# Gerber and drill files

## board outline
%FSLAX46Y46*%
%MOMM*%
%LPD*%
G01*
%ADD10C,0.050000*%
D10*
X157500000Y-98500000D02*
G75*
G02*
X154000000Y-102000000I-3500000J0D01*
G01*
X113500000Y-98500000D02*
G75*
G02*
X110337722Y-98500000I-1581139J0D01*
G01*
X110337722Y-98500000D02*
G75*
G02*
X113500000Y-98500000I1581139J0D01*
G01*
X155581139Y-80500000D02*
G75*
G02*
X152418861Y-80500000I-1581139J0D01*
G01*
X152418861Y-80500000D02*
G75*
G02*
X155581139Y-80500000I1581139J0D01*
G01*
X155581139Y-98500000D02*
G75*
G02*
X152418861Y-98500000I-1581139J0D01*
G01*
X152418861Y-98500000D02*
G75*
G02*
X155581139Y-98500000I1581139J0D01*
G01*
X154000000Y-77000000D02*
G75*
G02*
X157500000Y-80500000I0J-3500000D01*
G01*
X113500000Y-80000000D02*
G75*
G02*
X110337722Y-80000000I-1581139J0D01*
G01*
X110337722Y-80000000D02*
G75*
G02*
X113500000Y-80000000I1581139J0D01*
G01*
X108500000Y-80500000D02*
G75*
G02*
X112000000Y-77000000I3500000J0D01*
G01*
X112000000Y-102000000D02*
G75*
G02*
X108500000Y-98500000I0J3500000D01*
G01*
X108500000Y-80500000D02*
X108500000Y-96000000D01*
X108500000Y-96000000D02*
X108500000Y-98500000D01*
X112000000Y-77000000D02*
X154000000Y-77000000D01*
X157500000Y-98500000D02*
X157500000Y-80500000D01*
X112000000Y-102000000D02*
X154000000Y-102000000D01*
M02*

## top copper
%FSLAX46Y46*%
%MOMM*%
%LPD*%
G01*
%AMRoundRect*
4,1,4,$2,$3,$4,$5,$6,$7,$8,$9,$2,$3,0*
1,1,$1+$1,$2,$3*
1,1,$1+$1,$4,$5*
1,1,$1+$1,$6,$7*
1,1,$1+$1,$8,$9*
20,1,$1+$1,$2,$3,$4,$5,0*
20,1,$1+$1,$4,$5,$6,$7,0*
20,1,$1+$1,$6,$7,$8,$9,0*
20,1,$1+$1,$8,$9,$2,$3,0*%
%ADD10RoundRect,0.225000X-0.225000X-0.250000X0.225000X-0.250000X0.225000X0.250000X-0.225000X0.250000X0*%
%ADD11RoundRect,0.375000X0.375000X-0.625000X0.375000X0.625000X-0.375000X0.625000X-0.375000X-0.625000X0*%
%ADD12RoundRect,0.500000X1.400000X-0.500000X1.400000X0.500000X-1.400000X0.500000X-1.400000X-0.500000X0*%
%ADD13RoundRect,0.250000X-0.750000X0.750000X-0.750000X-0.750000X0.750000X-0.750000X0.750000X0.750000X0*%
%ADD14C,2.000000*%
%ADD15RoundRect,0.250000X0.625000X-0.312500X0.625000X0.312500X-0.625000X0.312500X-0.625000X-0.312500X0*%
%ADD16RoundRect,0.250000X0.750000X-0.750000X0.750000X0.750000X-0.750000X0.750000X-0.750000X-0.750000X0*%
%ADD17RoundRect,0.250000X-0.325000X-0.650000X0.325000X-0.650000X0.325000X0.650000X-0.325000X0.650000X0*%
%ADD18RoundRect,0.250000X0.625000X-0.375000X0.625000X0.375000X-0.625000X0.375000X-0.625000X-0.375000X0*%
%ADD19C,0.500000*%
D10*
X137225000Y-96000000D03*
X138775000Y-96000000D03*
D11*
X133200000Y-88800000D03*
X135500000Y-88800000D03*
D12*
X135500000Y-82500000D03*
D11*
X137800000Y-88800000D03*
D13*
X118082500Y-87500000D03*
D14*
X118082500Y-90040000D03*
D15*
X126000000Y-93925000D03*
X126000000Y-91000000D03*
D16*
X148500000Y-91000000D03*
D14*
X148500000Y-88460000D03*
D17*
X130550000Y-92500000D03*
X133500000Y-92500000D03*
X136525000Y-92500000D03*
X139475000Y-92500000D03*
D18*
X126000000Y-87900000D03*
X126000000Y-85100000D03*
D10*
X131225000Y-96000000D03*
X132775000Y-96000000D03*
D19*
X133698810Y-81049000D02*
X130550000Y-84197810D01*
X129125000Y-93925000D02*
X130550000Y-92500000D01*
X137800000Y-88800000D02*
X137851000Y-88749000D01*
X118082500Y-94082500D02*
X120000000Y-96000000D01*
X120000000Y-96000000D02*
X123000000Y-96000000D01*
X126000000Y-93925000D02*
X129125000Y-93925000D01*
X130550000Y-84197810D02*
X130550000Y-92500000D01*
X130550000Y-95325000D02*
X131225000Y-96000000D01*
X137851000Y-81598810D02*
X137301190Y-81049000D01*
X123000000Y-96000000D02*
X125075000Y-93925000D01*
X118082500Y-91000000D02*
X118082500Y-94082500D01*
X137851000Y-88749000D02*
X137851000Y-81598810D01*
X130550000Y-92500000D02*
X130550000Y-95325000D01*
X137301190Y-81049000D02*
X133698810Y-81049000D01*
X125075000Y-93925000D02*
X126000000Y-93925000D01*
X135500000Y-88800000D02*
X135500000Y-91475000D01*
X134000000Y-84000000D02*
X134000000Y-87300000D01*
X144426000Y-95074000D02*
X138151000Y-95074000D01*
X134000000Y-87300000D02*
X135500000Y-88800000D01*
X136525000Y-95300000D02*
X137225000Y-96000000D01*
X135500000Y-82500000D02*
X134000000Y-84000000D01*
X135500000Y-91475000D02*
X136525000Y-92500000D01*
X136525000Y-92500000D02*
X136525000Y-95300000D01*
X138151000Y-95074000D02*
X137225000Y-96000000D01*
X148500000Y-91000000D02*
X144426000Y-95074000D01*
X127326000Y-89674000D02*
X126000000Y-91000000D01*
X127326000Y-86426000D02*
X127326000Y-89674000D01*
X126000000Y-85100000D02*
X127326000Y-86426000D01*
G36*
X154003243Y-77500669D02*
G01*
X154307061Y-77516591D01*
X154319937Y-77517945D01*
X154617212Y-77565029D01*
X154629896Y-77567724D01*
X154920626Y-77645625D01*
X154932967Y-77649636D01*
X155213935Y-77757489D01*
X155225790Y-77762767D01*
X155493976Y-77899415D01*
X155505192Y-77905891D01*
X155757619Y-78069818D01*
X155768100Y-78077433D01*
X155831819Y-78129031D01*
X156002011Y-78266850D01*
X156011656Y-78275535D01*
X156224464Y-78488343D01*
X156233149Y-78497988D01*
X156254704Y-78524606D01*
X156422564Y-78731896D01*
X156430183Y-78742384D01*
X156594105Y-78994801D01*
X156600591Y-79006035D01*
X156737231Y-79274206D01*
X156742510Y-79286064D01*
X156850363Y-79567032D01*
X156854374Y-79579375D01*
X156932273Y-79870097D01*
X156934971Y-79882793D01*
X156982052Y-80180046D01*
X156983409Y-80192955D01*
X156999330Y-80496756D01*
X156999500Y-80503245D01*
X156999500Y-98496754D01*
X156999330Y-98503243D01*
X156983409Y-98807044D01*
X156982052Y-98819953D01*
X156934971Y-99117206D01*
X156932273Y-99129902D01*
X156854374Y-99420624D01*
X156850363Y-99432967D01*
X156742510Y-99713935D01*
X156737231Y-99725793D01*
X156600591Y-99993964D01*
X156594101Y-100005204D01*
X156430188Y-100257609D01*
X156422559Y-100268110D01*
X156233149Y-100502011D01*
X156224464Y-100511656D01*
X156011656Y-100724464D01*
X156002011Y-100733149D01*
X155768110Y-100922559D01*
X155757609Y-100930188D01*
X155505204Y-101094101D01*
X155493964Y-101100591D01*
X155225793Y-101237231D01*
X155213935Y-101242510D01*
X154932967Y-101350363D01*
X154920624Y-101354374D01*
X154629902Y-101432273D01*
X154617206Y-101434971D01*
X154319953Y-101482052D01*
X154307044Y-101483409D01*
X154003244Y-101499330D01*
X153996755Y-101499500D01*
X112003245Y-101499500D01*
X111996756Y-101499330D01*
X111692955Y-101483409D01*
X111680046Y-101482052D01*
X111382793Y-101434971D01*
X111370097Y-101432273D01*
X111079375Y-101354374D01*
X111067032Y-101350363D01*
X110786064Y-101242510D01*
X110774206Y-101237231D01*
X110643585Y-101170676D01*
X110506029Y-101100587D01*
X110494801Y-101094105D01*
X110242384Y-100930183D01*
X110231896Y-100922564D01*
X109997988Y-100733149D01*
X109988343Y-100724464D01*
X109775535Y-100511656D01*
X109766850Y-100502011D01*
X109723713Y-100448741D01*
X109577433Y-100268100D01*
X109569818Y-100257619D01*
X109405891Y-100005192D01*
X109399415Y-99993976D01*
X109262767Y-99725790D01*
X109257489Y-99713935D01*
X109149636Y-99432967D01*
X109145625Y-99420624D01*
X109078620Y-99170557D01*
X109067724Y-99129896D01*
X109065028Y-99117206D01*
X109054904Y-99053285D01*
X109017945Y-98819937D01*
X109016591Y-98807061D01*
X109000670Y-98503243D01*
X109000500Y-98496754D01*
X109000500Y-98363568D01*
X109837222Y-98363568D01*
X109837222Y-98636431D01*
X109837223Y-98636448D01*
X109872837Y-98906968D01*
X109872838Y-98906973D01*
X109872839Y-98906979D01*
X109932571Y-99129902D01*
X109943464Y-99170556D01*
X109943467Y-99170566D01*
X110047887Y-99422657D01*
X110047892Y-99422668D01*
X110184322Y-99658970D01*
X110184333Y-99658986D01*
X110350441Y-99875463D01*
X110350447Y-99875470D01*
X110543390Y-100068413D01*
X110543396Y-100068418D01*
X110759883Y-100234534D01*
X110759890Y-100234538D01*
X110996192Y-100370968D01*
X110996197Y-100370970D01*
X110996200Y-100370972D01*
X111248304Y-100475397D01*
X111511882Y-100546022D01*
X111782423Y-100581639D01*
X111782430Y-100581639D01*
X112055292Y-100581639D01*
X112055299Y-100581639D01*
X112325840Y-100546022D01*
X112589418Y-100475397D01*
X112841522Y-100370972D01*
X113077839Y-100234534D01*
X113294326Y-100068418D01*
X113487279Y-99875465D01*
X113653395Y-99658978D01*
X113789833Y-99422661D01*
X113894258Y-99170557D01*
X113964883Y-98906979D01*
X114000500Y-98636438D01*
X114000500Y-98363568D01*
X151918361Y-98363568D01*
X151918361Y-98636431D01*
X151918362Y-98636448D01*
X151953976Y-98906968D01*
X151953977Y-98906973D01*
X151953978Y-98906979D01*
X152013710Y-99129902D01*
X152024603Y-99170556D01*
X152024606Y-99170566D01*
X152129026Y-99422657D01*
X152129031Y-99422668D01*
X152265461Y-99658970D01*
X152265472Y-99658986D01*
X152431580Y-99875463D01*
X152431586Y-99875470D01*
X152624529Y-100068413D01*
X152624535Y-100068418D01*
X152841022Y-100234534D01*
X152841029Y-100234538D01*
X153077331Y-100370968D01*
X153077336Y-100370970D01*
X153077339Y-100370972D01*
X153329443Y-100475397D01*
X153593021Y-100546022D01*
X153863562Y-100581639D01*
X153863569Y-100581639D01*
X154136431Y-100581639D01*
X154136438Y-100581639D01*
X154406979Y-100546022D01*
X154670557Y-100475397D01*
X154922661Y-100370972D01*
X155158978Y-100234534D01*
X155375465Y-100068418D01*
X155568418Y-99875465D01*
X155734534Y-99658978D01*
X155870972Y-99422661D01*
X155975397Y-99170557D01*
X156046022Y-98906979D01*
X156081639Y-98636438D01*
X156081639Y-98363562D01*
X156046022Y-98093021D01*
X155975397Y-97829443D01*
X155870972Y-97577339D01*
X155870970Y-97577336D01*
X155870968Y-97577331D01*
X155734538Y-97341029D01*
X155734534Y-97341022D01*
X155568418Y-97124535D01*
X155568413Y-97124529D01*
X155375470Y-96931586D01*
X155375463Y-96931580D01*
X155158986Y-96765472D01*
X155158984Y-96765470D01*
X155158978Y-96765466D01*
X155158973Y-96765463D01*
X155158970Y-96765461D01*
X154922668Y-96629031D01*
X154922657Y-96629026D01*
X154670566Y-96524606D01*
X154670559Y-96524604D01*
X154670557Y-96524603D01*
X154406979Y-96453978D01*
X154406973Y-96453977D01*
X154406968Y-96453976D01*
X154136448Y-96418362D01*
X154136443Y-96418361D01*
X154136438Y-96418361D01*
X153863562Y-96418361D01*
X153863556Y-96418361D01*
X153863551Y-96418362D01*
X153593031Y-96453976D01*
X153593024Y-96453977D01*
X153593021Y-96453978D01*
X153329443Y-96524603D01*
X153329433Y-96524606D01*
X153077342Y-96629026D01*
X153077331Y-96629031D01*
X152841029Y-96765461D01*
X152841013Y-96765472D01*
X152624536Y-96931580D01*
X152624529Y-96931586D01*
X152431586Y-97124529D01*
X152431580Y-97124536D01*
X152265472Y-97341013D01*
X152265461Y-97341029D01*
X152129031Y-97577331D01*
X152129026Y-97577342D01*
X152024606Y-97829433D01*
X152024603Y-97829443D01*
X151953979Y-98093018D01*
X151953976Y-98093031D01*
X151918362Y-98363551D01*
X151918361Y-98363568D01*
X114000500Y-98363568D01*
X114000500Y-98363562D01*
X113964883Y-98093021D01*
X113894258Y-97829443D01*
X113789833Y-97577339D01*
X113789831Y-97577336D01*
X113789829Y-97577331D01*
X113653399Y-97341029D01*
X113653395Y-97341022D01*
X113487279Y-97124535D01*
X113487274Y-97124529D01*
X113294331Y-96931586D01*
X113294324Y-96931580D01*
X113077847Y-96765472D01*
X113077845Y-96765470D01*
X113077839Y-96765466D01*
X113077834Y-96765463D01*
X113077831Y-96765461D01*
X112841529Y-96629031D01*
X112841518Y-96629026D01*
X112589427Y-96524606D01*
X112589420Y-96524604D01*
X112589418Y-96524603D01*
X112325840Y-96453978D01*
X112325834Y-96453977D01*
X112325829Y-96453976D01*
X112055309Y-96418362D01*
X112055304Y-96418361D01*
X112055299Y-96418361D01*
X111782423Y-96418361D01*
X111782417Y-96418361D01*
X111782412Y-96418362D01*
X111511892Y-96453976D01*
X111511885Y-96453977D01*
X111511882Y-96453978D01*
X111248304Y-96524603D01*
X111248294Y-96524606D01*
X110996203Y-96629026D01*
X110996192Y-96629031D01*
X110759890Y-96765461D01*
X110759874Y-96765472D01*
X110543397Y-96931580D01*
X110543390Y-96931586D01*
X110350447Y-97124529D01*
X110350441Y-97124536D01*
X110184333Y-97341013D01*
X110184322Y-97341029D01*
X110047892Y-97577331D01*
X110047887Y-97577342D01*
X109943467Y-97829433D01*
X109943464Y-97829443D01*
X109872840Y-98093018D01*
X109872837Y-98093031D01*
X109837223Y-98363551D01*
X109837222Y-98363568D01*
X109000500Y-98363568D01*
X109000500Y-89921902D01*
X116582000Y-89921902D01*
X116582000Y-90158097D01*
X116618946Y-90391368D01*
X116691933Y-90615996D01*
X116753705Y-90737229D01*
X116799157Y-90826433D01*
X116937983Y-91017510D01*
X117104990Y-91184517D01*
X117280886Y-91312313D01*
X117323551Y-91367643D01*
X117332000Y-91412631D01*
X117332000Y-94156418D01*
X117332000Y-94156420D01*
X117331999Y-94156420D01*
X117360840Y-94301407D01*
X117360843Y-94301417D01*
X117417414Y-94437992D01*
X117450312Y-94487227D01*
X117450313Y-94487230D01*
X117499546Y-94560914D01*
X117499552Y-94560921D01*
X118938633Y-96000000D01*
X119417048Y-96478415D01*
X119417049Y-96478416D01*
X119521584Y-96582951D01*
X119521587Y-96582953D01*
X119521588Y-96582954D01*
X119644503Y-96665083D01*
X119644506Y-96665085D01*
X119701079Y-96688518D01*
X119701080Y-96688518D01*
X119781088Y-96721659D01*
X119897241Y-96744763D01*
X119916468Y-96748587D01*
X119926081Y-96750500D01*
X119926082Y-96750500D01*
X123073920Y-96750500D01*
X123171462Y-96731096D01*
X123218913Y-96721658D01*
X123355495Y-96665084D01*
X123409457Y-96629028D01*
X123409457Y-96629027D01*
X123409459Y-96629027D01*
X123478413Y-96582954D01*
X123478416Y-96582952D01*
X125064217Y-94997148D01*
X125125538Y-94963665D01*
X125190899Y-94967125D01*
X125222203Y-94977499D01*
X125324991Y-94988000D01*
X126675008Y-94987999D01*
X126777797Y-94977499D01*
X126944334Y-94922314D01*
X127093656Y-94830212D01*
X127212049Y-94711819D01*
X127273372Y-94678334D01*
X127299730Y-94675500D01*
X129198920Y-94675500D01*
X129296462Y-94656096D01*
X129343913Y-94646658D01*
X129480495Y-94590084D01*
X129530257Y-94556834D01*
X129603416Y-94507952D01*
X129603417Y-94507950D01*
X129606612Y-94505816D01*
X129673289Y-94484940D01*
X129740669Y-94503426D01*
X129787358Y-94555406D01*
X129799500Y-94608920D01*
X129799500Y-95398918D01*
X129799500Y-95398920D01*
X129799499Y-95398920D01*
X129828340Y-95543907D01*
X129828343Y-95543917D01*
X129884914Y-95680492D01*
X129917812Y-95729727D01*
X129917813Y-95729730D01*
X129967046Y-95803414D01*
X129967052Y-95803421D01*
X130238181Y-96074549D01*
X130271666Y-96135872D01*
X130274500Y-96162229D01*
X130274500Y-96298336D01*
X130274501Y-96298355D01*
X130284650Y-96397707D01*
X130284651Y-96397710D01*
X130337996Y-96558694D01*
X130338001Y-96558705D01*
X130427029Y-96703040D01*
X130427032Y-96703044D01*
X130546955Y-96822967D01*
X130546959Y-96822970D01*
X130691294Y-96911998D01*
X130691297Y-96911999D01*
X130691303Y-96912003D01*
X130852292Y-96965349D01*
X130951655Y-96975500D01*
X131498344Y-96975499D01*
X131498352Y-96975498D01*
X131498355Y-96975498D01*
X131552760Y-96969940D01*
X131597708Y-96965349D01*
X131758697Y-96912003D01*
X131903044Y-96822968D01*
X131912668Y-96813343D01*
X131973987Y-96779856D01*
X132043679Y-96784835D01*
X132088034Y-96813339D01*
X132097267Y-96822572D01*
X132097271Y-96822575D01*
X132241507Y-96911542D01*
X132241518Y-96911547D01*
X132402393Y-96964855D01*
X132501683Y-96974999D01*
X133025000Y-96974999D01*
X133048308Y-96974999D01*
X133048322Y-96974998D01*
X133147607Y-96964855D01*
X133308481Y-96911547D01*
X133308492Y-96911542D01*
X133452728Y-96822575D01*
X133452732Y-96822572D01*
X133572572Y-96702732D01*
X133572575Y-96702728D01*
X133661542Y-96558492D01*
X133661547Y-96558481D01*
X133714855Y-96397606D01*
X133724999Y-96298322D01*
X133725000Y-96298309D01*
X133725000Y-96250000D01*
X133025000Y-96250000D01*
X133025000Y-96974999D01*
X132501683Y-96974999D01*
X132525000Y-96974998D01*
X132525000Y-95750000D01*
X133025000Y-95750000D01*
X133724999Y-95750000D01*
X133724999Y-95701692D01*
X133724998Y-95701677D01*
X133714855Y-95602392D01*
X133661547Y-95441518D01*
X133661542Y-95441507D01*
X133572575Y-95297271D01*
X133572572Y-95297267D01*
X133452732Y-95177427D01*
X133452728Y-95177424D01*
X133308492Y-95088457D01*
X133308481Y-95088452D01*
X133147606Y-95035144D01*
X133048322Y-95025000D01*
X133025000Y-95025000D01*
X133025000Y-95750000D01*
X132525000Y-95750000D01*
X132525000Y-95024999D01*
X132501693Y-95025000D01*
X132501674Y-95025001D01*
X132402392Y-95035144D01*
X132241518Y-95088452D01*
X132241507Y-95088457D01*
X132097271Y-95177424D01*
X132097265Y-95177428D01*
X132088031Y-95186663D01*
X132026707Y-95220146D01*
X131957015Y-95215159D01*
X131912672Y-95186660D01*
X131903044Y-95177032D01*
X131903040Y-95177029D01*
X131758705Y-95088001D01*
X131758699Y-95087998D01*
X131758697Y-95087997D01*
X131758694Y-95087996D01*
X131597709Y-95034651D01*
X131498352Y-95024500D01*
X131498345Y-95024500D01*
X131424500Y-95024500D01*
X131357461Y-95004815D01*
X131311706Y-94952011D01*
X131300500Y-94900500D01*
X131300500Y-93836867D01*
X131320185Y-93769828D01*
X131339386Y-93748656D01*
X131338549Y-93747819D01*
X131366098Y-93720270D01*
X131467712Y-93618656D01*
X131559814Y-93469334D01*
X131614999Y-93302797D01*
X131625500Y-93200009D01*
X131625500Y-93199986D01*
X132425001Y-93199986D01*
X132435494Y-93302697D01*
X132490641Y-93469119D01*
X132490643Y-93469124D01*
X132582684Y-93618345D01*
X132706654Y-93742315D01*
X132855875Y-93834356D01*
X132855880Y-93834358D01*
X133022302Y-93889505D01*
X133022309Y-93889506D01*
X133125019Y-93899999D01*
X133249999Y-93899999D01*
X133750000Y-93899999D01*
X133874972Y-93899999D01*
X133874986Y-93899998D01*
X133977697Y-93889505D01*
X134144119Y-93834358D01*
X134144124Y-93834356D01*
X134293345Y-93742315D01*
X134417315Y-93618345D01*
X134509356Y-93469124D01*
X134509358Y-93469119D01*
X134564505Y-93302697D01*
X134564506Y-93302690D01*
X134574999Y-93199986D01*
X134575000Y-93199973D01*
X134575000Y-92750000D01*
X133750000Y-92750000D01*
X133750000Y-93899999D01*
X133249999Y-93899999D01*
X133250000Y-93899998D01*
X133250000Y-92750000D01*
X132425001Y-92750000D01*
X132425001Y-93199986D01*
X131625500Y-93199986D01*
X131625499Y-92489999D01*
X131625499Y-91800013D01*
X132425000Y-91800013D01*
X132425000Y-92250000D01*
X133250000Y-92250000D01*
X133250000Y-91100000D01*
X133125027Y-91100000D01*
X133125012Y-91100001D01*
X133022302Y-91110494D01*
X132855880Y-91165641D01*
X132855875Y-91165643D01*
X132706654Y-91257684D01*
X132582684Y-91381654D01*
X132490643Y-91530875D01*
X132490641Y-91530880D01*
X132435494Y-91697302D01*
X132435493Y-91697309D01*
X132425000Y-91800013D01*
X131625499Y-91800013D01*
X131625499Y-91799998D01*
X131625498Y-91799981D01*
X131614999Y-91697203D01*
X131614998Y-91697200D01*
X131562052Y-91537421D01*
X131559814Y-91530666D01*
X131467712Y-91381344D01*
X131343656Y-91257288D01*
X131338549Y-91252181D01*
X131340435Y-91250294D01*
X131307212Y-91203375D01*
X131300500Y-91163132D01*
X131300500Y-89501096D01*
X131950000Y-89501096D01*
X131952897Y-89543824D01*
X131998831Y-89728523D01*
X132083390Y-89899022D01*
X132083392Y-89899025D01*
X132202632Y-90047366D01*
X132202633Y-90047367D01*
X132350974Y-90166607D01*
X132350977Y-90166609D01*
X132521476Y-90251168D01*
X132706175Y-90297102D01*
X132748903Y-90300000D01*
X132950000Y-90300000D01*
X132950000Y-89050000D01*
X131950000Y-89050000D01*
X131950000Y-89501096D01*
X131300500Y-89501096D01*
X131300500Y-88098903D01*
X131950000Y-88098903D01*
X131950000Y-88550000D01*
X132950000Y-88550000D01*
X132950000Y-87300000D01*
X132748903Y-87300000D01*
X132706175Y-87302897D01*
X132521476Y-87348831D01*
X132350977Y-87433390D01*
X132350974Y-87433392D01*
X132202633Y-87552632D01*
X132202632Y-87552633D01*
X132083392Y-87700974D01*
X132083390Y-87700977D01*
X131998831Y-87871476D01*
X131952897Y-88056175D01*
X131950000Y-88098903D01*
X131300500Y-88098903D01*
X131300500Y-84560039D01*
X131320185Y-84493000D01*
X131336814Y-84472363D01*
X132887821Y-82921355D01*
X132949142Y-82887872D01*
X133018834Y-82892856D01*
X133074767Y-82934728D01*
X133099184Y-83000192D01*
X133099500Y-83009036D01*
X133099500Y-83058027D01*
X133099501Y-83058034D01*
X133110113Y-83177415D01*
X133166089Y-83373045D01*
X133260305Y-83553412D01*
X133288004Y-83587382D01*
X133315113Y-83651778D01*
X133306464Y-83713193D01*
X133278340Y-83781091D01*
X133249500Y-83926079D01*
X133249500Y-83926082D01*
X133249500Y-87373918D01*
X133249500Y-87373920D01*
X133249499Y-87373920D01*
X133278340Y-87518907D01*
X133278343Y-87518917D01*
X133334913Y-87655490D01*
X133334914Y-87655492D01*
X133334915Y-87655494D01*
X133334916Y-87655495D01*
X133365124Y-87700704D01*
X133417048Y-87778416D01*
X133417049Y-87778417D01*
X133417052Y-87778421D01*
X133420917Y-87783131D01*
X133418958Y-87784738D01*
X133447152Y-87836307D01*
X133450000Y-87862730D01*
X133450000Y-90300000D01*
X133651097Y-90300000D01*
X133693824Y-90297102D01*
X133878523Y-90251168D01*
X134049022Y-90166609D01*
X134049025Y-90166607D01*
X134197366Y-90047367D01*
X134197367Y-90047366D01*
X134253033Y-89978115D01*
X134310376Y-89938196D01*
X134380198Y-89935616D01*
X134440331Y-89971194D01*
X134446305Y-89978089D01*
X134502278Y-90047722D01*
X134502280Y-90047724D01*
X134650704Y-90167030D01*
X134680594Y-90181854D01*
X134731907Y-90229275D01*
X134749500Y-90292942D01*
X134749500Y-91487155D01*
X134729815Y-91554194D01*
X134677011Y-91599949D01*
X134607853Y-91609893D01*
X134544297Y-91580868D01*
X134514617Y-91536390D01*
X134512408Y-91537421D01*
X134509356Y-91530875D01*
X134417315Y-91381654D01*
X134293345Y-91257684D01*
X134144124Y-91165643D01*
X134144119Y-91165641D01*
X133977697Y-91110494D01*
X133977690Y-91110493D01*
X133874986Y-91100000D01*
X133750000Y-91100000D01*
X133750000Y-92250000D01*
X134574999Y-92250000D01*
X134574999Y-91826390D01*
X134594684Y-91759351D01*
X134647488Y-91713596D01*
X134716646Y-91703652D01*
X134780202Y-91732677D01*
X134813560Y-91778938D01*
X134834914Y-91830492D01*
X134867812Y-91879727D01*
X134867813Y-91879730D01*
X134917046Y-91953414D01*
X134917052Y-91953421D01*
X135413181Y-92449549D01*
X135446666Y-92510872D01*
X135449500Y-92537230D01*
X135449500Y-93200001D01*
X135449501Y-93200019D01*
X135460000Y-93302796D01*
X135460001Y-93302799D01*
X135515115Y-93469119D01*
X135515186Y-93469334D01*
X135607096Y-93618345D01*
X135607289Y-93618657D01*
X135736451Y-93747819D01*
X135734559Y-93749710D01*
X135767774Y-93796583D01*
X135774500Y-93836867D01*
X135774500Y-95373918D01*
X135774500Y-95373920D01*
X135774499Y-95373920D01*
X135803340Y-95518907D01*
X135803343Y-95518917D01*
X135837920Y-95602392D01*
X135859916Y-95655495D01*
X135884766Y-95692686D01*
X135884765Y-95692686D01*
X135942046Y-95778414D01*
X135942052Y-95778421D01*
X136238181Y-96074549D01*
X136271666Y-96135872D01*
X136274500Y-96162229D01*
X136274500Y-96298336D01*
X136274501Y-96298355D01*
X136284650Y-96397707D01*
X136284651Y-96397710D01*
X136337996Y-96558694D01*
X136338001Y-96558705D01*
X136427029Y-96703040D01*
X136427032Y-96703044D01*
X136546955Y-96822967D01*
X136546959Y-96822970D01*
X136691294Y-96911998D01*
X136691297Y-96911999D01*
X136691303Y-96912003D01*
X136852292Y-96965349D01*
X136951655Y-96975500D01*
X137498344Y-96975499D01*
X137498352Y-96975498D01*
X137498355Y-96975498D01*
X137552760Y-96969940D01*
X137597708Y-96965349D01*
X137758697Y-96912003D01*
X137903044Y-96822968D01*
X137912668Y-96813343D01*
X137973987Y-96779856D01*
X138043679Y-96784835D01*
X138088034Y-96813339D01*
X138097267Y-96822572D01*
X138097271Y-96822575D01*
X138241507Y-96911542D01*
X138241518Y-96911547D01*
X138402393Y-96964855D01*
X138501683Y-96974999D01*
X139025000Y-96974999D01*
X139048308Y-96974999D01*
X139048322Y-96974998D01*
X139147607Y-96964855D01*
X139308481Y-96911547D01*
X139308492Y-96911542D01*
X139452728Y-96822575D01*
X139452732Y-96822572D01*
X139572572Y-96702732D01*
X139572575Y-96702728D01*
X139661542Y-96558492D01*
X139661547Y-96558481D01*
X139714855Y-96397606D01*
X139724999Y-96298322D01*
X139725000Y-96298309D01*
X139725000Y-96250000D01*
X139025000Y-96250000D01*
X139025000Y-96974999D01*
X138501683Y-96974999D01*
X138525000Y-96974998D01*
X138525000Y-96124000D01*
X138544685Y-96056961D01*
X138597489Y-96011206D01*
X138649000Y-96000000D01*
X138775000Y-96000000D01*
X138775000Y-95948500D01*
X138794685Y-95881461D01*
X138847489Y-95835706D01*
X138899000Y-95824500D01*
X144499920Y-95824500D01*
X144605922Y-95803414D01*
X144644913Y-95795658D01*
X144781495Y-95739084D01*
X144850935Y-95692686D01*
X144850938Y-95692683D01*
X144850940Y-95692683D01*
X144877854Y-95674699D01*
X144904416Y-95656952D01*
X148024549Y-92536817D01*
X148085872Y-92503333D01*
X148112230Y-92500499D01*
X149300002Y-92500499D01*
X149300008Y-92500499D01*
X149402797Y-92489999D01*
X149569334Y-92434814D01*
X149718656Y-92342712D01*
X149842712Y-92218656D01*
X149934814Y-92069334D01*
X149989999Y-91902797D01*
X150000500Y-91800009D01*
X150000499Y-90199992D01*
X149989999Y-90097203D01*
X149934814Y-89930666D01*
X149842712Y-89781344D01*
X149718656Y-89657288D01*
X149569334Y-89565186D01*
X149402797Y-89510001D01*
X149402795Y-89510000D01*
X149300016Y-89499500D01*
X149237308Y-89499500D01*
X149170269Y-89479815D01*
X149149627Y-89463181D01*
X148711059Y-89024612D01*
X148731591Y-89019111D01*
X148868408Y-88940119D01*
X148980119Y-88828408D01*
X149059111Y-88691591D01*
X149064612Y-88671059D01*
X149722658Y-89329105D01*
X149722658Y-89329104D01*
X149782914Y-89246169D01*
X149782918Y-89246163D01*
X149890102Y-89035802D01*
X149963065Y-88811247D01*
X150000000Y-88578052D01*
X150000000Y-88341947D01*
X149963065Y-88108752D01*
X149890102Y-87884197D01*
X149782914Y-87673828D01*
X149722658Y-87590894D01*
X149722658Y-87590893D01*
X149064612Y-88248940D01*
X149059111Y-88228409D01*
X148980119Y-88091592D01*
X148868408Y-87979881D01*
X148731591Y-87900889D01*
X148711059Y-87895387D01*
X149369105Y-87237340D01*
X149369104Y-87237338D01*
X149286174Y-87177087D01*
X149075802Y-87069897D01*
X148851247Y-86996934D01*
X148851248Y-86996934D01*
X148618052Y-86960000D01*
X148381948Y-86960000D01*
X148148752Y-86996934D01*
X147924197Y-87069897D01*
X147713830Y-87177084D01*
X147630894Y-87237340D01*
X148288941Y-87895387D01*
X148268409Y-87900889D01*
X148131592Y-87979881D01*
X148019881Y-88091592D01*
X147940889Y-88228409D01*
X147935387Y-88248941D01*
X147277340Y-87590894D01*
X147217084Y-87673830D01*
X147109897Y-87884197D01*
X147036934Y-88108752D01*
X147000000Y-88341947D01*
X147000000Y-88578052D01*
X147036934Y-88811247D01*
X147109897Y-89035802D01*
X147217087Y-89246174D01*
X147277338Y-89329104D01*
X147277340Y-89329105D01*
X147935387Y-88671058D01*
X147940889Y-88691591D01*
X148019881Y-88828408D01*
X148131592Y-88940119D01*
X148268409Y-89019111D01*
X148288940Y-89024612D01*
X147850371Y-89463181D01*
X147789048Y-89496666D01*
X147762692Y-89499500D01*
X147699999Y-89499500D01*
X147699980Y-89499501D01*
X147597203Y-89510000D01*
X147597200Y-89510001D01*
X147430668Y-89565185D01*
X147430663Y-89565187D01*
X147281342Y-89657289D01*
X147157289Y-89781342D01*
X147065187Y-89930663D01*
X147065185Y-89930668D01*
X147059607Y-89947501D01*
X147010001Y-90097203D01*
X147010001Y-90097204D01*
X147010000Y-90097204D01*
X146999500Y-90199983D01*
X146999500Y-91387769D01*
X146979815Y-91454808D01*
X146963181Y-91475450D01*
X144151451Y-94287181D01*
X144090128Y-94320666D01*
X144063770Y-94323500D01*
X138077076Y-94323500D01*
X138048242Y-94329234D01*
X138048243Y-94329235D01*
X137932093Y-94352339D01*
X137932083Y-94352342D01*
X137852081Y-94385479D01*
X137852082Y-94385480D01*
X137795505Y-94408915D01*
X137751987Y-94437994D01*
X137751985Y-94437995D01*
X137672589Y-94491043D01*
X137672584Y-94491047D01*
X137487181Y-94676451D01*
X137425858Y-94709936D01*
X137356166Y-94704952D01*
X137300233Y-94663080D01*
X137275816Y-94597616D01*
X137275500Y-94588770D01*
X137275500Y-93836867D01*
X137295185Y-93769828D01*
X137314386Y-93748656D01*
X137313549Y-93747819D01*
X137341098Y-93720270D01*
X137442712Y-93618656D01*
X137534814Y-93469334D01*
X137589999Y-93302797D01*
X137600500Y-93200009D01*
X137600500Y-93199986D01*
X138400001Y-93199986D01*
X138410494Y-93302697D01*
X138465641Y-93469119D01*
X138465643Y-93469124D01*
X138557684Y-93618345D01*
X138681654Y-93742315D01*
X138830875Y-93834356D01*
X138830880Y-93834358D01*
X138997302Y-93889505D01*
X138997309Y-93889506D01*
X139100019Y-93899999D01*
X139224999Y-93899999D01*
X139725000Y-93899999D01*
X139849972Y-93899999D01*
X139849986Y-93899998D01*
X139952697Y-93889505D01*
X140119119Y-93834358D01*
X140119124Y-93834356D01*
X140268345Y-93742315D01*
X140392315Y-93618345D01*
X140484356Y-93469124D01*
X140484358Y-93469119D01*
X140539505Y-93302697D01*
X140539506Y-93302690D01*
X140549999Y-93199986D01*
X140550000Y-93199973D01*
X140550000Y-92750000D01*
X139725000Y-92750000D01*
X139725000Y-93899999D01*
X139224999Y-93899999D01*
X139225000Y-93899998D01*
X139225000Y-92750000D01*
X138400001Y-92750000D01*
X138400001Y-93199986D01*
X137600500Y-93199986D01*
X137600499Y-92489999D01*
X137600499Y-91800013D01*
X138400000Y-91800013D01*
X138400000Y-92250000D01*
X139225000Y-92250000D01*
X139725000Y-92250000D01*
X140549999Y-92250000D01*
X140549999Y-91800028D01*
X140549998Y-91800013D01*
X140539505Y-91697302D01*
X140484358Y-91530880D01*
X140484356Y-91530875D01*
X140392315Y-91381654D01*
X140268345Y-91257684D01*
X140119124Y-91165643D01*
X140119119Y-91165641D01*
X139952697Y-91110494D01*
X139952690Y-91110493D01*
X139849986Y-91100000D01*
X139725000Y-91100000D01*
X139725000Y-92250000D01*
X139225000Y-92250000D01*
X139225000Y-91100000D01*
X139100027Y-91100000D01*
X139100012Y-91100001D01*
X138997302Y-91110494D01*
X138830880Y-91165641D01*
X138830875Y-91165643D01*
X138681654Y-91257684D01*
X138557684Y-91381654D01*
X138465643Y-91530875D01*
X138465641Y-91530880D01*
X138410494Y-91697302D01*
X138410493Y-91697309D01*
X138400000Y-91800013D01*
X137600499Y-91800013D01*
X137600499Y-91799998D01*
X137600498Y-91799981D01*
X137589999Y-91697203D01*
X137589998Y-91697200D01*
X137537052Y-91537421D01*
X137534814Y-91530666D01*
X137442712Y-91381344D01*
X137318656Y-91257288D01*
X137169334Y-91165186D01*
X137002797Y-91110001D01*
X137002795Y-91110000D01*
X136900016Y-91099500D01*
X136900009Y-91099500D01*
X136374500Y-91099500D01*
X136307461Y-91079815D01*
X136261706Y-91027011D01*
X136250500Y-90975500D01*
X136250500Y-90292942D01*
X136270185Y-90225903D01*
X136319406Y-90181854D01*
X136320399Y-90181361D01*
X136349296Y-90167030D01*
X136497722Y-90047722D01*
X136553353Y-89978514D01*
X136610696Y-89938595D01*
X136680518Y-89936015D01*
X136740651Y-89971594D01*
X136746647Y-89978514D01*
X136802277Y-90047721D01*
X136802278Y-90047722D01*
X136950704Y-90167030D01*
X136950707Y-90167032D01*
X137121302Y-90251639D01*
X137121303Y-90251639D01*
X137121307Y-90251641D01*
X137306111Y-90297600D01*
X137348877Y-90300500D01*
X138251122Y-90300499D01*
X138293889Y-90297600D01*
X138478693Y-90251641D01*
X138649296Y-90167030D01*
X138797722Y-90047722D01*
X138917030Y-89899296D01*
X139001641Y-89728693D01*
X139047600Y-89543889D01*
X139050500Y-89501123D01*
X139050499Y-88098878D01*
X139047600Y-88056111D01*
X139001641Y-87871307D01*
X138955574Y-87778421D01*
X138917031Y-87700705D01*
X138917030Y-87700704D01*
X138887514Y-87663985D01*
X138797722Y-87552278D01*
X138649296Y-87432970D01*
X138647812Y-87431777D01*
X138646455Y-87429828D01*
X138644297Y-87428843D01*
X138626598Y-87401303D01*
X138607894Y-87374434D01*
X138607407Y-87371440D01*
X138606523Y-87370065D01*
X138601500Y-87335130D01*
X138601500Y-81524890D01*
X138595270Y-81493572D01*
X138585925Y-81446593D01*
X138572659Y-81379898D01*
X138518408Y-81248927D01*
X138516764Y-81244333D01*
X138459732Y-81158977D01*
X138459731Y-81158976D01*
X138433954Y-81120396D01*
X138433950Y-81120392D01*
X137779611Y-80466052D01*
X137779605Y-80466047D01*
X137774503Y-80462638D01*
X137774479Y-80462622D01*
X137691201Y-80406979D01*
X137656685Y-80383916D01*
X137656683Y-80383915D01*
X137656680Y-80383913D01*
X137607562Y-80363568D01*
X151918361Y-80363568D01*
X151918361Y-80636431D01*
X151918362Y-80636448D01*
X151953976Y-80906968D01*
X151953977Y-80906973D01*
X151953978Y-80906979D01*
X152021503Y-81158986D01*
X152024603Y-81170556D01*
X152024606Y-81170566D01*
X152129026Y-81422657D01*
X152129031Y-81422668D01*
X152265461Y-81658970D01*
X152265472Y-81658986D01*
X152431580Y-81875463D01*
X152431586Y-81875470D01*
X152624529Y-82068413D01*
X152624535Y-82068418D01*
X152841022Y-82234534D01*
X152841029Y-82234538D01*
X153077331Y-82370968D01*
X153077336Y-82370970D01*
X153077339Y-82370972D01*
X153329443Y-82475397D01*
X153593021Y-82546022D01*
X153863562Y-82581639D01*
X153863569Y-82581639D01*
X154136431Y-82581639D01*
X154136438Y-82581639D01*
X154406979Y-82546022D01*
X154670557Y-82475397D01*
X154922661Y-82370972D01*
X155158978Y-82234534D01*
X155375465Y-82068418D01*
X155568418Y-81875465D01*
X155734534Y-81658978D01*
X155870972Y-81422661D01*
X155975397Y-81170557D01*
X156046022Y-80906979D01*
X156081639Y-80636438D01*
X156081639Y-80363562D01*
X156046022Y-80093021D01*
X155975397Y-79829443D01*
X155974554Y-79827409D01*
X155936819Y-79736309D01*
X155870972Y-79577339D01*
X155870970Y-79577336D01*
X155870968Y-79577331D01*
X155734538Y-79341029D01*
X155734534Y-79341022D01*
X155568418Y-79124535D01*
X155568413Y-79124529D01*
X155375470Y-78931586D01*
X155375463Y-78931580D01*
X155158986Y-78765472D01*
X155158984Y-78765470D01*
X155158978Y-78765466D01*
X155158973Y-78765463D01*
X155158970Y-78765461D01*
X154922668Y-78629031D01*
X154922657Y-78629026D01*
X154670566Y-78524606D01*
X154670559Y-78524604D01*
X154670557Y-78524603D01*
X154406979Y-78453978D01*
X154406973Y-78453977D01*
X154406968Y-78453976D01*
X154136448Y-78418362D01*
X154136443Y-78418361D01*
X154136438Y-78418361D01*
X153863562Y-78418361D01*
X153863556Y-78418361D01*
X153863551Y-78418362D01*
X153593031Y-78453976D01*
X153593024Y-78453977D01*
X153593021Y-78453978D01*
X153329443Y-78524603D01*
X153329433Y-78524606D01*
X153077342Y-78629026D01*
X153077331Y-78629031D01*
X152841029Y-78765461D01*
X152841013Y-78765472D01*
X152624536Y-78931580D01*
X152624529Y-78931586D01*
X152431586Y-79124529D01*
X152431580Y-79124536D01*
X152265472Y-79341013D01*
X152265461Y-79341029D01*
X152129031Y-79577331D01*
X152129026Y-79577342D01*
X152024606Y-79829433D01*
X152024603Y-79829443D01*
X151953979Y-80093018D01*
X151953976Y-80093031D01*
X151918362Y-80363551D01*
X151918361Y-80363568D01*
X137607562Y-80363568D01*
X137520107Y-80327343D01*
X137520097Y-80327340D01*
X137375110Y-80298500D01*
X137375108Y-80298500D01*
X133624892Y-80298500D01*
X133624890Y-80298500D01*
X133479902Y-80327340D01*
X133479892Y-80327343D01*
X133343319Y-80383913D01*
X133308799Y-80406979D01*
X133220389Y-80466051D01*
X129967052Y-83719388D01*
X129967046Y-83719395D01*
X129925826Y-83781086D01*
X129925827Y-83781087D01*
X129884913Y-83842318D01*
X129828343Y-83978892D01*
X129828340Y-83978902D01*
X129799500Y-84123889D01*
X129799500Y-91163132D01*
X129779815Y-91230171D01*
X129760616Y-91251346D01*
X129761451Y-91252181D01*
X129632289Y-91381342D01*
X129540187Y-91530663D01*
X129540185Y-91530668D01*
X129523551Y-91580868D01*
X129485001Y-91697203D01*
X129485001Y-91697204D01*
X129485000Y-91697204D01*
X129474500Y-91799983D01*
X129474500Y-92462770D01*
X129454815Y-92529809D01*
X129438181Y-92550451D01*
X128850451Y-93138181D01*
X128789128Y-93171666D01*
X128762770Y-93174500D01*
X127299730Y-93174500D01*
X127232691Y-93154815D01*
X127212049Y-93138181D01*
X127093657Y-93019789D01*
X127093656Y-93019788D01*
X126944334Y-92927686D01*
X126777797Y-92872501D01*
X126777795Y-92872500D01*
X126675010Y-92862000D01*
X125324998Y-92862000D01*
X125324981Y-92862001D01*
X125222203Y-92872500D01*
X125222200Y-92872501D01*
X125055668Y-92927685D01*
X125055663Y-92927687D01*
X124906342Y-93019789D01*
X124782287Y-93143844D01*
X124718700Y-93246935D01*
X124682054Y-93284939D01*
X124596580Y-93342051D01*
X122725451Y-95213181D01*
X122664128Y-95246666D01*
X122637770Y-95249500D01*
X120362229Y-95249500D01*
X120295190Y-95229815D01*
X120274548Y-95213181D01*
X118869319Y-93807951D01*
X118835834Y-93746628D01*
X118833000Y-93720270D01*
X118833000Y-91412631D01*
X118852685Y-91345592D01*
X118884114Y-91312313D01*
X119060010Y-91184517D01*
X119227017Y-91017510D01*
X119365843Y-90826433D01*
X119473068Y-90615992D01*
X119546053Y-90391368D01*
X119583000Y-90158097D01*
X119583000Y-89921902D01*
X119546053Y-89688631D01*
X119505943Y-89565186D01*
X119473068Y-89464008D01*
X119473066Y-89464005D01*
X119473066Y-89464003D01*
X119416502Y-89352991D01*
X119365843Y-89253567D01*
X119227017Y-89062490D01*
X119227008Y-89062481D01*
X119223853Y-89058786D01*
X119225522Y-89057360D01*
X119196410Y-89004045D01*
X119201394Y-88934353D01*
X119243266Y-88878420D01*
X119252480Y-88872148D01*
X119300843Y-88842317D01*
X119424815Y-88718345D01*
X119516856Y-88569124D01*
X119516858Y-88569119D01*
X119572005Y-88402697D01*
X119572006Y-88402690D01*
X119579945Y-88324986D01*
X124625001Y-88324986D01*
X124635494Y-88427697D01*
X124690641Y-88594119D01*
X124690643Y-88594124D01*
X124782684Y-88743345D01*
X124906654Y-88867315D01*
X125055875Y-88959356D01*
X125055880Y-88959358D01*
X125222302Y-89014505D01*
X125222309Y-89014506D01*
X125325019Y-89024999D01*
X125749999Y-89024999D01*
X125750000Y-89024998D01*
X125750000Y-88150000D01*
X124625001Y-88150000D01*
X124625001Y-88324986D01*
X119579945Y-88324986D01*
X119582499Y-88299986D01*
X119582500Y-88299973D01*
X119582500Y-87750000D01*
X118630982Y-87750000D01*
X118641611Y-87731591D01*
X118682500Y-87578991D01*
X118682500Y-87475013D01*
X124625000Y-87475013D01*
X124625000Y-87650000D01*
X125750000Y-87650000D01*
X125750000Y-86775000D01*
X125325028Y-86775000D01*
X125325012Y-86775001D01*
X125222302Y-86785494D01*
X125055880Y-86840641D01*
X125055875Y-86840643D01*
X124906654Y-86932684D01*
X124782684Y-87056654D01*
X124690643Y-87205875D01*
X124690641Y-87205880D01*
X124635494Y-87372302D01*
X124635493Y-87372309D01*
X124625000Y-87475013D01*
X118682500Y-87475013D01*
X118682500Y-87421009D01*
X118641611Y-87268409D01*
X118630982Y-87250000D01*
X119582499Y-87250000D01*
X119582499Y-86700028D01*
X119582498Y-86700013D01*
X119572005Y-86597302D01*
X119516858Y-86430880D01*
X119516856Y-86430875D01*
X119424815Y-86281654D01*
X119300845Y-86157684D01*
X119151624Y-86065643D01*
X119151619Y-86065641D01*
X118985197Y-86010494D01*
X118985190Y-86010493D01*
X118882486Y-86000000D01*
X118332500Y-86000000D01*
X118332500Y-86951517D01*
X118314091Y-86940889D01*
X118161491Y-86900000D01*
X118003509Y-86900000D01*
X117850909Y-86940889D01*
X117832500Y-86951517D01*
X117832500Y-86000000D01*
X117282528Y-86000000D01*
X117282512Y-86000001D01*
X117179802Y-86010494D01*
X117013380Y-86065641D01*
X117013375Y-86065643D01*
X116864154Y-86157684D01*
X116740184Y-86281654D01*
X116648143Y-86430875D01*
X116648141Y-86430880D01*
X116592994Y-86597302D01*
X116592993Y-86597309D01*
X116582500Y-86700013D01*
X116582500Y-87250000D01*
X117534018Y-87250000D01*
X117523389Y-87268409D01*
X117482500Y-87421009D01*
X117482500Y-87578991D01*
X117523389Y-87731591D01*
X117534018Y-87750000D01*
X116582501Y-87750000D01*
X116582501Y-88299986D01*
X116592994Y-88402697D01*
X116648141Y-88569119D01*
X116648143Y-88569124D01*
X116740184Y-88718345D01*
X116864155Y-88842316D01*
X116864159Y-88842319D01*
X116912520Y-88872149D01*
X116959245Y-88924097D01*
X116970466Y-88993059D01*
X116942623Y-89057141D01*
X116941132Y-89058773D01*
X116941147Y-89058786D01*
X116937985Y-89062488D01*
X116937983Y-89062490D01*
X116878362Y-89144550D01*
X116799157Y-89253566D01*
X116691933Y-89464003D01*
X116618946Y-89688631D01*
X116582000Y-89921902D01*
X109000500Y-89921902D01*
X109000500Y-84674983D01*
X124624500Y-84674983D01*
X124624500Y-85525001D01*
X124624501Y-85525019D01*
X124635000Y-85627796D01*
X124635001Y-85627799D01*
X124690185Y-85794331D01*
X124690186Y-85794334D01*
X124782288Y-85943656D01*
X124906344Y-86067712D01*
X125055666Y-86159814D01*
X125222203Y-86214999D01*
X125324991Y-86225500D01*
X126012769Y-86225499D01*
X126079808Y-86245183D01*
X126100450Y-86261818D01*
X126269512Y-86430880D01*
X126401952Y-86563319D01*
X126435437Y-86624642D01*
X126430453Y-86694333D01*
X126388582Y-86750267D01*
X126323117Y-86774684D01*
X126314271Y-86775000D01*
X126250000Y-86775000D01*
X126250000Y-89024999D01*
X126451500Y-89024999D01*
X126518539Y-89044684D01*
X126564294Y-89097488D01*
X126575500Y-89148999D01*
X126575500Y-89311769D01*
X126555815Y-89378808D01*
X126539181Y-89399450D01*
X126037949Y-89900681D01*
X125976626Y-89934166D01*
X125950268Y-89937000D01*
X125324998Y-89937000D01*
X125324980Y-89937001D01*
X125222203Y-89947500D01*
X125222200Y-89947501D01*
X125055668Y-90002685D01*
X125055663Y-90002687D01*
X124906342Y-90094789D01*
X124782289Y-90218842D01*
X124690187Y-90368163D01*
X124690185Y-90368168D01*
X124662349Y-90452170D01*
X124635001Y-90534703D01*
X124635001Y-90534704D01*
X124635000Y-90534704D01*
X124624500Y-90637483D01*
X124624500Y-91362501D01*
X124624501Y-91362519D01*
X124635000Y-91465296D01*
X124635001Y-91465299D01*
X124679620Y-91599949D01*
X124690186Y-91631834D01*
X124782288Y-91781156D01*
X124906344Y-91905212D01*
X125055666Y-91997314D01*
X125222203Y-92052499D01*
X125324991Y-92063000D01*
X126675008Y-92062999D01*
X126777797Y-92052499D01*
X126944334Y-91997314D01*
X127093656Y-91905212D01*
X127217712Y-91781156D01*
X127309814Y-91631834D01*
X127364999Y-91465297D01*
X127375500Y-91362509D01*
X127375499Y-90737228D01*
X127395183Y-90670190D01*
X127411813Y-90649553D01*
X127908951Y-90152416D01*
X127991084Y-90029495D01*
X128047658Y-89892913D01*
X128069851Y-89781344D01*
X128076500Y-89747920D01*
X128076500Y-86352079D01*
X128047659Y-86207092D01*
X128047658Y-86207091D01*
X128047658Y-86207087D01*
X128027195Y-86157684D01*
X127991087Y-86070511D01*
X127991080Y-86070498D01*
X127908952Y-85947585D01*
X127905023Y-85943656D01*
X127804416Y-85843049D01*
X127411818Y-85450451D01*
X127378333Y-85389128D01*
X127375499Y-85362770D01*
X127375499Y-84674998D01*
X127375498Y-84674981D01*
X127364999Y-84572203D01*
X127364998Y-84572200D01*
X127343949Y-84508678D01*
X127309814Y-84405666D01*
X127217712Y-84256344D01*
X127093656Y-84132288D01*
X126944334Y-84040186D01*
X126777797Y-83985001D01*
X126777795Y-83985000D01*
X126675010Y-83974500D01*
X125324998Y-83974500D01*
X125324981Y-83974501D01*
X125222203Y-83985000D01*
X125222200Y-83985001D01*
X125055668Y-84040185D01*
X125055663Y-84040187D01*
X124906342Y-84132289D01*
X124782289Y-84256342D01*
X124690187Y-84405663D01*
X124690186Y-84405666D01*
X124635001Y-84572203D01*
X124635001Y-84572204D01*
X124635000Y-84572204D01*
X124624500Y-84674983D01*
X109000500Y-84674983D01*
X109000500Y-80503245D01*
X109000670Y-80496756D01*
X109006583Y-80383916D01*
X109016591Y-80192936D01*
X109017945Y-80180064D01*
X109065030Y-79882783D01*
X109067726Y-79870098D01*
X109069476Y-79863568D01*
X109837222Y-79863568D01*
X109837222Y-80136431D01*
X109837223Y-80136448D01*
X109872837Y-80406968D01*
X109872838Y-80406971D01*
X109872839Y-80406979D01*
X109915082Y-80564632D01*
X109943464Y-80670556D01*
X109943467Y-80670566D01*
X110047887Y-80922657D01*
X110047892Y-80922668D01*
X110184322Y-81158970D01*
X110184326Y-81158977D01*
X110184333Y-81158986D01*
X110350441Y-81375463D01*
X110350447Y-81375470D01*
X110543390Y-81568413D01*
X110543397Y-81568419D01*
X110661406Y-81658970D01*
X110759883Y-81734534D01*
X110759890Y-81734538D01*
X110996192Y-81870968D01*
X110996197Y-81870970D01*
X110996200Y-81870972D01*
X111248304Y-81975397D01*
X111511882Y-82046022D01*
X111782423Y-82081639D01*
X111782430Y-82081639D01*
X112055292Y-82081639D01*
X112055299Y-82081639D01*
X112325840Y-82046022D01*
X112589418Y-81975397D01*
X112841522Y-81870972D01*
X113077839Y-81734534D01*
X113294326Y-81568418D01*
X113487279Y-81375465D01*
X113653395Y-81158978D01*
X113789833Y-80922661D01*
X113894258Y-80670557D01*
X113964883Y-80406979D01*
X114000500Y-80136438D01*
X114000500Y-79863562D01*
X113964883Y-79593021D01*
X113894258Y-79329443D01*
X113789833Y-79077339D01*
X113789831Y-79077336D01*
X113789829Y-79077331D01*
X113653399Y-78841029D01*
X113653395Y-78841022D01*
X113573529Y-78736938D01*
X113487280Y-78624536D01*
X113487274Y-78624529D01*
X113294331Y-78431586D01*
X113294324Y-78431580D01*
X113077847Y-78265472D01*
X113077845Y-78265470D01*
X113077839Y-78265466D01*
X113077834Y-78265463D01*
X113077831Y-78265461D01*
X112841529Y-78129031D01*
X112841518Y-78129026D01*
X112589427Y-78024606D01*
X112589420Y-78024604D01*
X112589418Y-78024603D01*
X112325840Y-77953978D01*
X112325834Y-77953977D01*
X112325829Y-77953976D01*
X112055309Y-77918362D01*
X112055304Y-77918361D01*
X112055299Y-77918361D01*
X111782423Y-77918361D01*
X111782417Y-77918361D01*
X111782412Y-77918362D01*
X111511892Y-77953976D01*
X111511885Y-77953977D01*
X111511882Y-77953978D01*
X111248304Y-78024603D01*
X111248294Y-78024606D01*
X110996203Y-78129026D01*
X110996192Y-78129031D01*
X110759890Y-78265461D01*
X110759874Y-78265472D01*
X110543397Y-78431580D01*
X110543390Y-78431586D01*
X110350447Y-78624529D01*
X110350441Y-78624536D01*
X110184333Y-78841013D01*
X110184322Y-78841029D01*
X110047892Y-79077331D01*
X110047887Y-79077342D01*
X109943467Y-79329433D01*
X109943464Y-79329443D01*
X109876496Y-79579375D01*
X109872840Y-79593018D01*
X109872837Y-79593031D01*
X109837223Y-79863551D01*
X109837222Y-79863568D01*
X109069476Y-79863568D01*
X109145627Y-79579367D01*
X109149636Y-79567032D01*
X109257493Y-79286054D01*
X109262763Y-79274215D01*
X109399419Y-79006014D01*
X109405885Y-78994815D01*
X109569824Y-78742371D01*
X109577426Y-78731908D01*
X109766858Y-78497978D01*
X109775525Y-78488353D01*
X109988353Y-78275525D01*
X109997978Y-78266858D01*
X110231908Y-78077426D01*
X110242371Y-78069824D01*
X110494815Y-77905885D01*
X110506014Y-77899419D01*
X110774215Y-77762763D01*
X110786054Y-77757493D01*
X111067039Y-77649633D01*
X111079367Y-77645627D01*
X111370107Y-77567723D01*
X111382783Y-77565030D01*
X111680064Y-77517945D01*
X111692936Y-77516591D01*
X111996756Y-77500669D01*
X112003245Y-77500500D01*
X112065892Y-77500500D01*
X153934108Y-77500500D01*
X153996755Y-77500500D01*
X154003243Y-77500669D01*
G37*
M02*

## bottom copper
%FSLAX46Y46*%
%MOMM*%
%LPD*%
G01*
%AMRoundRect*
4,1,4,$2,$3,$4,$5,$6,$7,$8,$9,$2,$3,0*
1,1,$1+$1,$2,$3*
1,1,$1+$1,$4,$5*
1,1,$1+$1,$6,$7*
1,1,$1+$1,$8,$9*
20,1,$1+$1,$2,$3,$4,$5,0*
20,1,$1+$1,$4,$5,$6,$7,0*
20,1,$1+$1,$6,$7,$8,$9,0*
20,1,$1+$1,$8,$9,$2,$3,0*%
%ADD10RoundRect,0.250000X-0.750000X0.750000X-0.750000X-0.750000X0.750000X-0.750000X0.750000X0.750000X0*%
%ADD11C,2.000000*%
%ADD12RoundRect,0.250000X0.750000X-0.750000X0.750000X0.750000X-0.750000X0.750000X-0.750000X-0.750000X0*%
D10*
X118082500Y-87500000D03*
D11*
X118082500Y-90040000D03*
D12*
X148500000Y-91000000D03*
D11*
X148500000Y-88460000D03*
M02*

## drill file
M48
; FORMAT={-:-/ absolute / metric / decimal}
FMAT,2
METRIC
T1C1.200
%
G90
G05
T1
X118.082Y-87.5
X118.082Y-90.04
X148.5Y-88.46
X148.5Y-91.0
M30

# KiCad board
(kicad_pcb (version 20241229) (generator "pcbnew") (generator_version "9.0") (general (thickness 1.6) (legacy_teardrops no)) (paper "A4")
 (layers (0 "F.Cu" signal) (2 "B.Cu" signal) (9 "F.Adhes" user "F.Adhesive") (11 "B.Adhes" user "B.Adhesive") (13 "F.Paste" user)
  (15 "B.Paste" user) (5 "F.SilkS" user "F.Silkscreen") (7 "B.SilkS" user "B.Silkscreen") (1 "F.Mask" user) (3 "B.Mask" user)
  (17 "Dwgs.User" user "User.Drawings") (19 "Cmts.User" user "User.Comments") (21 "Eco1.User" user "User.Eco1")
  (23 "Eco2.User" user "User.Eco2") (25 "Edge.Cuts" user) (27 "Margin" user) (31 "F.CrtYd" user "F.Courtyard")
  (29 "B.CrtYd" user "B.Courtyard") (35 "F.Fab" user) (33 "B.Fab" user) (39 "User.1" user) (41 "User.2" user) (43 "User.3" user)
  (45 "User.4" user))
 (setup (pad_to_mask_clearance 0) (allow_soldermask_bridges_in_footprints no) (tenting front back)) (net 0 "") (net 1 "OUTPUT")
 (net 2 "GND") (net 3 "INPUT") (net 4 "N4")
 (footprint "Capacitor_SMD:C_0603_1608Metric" (layer "F.Cu") (at 138 96)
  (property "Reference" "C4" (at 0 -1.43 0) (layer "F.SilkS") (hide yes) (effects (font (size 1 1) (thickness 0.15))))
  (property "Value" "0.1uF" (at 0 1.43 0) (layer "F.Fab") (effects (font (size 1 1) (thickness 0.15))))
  (pad "1" smd roundrect (at -0.775 0) (size 0.9 0.95) (layers "F.Cu" "F.Mask" "F.Paste") (roundrect_rratio 0.25) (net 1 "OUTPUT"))
  (pad "2" smd roundrect (at 0.775 0) (size 0.9 0.95) (layers "F.Cu" "F.Mask" "F.Paste") (roundrect_rratio 0.25) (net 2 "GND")))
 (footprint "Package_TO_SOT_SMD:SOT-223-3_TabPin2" (layer "F.Cu") (at 135.5 85.65 90)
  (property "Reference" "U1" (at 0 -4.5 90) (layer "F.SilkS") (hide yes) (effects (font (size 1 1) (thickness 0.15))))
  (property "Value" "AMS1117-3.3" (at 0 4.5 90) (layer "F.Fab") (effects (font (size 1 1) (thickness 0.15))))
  (pad "1" smd roundrect (at -3.15 -2.3 90) (size 2 1.5) (layers "F.Cu" "F.Mask" "F.Paste") (roundrect_rratio 0.25) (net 2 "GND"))
  (pad "2" smd roundrect (at -3.15 0 90) (size 2 1.5) (layers "F.Cu" "F.Mask" "F.Paste") (roundrect_rratio 0.25) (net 1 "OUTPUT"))
  (pad "2" smd roundrect (at 3.15 0 90) (size 2 3.8) (layers "F.Cu" "F.Mask" "F.Paste") (roundrect_rratio 0.25) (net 1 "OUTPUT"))
  (pad "3" smd roundrect (at -3.15 2.3 90) (size 2 1.5) (layers "F.Cu" "F.Mask" "F.Paste") (roundrect_rratio 0.25) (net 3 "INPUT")))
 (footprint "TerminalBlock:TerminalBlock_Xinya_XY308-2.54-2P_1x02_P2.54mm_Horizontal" (layer "F.Cu") (at 118.0825 87.5 -90)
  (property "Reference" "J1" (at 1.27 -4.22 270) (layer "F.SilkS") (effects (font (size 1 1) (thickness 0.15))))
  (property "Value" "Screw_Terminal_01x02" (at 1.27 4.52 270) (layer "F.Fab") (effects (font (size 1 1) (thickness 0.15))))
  (pad "1" thru_hole roundrect (at 0 0 270) (size 2 2) (drill 1.2) (layers "*.Cu" "*.Mask") (remove_unused_layers no)
   (roundrect_rratio 0.125) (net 2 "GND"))
  (pad "2" thru_hole circle (at 2.54 0 270) (size 2 2) (drill 1.2) (layers "*.Cu" "*.Mask") (remove_unused_layers no) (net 3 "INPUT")))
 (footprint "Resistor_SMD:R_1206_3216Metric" (layer "F.Cu") (at 126 92.4625 90)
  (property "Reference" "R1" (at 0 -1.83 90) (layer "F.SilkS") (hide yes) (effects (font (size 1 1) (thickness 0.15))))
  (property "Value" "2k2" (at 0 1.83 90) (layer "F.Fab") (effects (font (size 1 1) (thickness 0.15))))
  (pad "1" smd roundrect (at -1.4625 0 90) (size 1.125 1.75) (layers "F.Cu" "F.Mask" "F.Paste") (roundrect_rratio 0.222222) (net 3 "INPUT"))
  (pad "2" smd roundrect (at 1.4625 0 90) (size 1.125 1.75) (layers "F.Cu" "F.Mask" "F.Paste") (roundrect_rratio 0.222222) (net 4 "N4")))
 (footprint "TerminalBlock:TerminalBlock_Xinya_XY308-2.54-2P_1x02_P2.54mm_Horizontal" (layer "F.Cu") (at 148.5 91 90)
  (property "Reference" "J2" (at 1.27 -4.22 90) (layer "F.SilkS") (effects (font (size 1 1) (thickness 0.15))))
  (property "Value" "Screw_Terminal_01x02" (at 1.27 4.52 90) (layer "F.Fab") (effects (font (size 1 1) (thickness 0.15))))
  (pad "1" thru_hole roundrect (at 0 0 90) (size 2 2) (drill 1.2) (layers "*.Cu" "*.Mask") (remove_unused_layers no)
   (roundrect_rratio 0.125) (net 1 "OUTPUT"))
  (pad "2" thru_hole circle (at 2.54 0 90) (size 2 2) (drill 1.2) (layers "*.Cu" "*.Mask") (remove_unused_layers no) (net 2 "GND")))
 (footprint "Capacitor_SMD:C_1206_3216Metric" (layer "F.Cu") (at 132.025 92.5)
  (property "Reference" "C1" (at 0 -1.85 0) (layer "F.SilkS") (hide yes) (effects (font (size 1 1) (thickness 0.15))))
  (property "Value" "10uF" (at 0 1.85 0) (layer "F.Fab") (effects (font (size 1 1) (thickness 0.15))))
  (pad "1" smd roundrect (at -1.475 0) (size 1.15 1.8) (layers "F.Cu" "F.Mask" "F.Paste") (roundrect_rratio 0.217391) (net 3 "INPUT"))
  (pad "2" smd roundrect (at 1.475 0) (size 1.15 1.8) (layers "F.Cu" "F.Mask" "F.Paste") (roundrect_rratio 0.217391) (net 2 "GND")))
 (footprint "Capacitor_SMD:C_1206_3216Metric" (layer "F.Cu") (at 138 92.5)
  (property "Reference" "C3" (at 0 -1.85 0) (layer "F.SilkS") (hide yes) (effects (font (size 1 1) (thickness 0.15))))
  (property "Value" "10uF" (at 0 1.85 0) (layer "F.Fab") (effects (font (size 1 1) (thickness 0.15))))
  (pad "1" smd roundrect (at -1.475 0) (size 1.15 1.8) (layers "F.Cu" "F.Mask" "F.Paste") (roundrect_rratio 0.217391) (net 1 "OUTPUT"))
  (pad "2" smd roundrect (at 1.475 0) (size 1.15 1.8) (layers "F.Cu" "F.Mask" "F.Paste") (roundrect_rratio 0.217391) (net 2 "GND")))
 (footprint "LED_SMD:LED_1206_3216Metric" (layer "F.Cu") (at 126 86.5 90)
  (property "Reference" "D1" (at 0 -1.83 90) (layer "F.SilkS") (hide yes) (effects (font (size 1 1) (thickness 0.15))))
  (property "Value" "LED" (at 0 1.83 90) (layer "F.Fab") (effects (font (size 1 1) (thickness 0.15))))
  (pad "1" smd roundrect (at -1.4 0 90) (size 1.25 1.75) (layers "F.Cu" "F.Mask" "F.Paste") (roundrect_rratio 0.2) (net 2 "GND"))
  (pad "2" smd roundrect (at 1.4 0 90) (size 1.25 1.75) (layers "F.Cu" "F.Mask" "F.Paste") (roundrect_rratio 0.2) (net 4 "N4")))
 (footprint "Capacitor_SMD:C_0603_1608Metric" (layer "F.Cu") (at 132 96)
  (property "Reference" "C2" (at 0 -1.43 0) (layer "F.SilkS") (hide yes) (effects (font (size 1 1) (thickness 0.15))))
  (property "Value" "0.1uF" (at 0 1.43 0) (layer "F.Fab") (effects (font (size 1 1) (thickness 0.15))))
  (pad "1" smd roundrect (at -0.775 0) (size 0.9 0.95) (layers "F.Cu" "F.Mask" "F.Paste") (roundrect_rratio 0.25) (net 3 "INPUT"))
  (pad "2" smd roundrect (at 0.775 0) (size 0.9 0.95) (layers "F.Cu" "F.Mask" "F.Paste") (roundrect_rratio 0.25) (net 2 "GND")))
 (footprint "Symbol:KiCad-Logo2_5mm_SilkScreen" (layer "B.Cu") (at 130 92 180)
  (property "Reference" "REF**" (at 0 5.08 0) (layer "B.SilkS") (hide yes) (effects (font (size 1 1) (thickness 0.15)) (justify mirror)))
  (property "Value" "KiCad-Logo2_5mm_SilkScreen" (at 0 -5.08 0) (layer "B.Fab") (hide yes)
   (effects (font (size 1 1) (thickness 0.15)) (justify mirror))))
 (gr_arc (start 157.5 98.5) (mid 156.474874 100.974874) (end 154 102) (stroke (width 0.05) (type default)) (layer "Edge.Cuts"))
 (gr_circle (center 111.918861 98.5) (end 113.418861 98) (stroke (width 0.05) (type default)) (fill no) (layer "Edge.Cuts"))
 (gr_circle (center 154 80.5) (end 155.5 80) (stroke (width 0.05) (type default)) (fill no) (layer "Edge.Cuts"))
 (gr_circle (center 154 98.5) (end 155.5 98) (stroke (width 0.05) (type default)) (fill no) (layer "Edge.Cuts"))
 (gr_arc (start 154 77) (mid 156.474874 78.025126) (end 157.5 80.5) (stroke (width 0.05) (type default)) (layer "Edge.Cuts"))
 (gr_circle (center 111.918861 80) (end 113.418861 79.5) (stroke (width 0.05) (type default)) (fill no) (layer "Edge.Cuts"))
 (gr_arc (start 108.5 80.5) (mid 109.525126 78.025126) (end 112 77) (stroke (width 0.05) (type default)) (layer "Edge.Cuts"))
 (gr_arc (start 112 102) (mid 109.525126 100.974874) (end 108.5 98.5) (stroke (width 0.05) (type default)) (layer "Edge.Cuts"))
 (gr_line (start 108.5 80.5) (end 108.5 96) (stroke (width 0.05) (type default)) (layer "Edge.Cuts"))
 (gr_line (start 108.5 96) (end 108.5 98.5) (stroke (width 0.05) (type default)) (layer "Edge.Cuts"))
 (gr_line (start 112 77) (end 154 77) (stroke (width 0.05) (type default)) (layer "Edge.Cuts"))
 (gr_line (start 157.5 98.5) (end 157.5 80.5) (stroke (width 0.05) (type default)) (layer "Edge.Cuts"))
 (gr_line (start 112 102) (end 154 102) (stroke (width 0.05) (type default)) (layer "Edge.Cuts"))
 (segment (start 133.69881 81.049) (end 130.55 84.19781) (width 0.5) (layer "F.Cu") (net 3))
 (segment (start 129.125 93.925) (end 130.55 92.5) (width 0.5) (layer "F.Cu") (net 3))
 (segment (start 137.8 88.8) (end 137.851 88.749) (width 0.5) (layer "F.Cu") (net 3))
 (segment (start 118.0825 94.0825) (end 120 96) (width 0.5) (layer "F.Cu") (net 3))
 (segment (start 120 96) (end 123 96) (width 0.5) (layer "F.Cu") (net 3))
 (segment (start 126 93.925) (end 129.125 93.925) (width 0.5) (layer "F.Cu") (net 3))
 (segment (start 130.55 84.19781) (end 130.55 92.5) (width 0.5) (layer "F.Cu") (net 3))
 (segment (start 130.55 95.325) (end 131.225 96) (width 0.5) (layer "F.Cu") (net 3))
 (segment (start 137.851 81.59881) (end 137.30119 81.049) (width 0.5) (layer "F.Cu") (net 3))
 (segment (start 123 96) (end 125.075 93.925) (width 0.5) (layer "F.Cu") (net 3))
 (segment (start 118.0825 91) (end 118.0825 94.0825) (width 0.5) (layer "F.Cu") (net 3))
 (segment (start 137.851 88.749) (end 137.851 81.59881) (width 0.5) (layer "F.Cu") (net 3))
 (segment (start 130.55 92.5) (end 130.55 95.325) (width 0.5) (layer "F.Cu") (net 3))
 (segment (start 137.30119 81.049) (end 133.69881 81.049) (width 0.5) (layer "F.Cu") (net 3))
 (segment (start 125.075 93.925) (end 126 93.925) (width 0.5) (layer "F.Cu") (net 3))
 (segment (start 135.5 88.8) (end 135.5 91.475) (width 0.5) (layer "F.Cu") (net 1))
 (segment (start 134 84) (end 134 87.3) (width 0.5) (layer "F.Cu") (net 1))
 (segment (start 144.426 95.074) (end 138.151 95.074) (width 0.5) (layer "F.Cu") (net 1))
 (segment (start 134 87.3) (end 135.5 88.8) (width 0.5) (layer "F.Cu") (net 1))
 (segment (start 136.525 95.3) (end 137.225 96) (width 0.5) (layer "F.Cu") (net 1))
 (segment (start 135.5 82.5) (end 134 84) (width 0.5) (layer "F.Cu") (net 1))
 (segment (start 135.5 91.475) (end 136.525 92.5) (width 0.5) (layer "F.Cu") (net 1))
 (segment (start 136.525 92.5) (end 136.525 95.3) (width 0.5) (layer "F.Cu") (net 1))
 (segment (start 138.151 95.074) (end 137.225 96) (width 0.5) (layer "F.Cu") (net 1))
 (segment (start 148.5 91) (end 144.426 95.074) (width 0.5) (layer "F.Cu") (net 1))
 (segment (start 127.326 89.674) (end 126 91) (width 0.5) (layer "F.Cu") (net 4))
 (segment (start 127.326 86.426) (end 127.326 89.674) (width 0.5) (layer "F.Cu") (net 4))
 (segment (start 126 85.1) (end 127.326 86.426) (width 0.5) (layer "F.Cu") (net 4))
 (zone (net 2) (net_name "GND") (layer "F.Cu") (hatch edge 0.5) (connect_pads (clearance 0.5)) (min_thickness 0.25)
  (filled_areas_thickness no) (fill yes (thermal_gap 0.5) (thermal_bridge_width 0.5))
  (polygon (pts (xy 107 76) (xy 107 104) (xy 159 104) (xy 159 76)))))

